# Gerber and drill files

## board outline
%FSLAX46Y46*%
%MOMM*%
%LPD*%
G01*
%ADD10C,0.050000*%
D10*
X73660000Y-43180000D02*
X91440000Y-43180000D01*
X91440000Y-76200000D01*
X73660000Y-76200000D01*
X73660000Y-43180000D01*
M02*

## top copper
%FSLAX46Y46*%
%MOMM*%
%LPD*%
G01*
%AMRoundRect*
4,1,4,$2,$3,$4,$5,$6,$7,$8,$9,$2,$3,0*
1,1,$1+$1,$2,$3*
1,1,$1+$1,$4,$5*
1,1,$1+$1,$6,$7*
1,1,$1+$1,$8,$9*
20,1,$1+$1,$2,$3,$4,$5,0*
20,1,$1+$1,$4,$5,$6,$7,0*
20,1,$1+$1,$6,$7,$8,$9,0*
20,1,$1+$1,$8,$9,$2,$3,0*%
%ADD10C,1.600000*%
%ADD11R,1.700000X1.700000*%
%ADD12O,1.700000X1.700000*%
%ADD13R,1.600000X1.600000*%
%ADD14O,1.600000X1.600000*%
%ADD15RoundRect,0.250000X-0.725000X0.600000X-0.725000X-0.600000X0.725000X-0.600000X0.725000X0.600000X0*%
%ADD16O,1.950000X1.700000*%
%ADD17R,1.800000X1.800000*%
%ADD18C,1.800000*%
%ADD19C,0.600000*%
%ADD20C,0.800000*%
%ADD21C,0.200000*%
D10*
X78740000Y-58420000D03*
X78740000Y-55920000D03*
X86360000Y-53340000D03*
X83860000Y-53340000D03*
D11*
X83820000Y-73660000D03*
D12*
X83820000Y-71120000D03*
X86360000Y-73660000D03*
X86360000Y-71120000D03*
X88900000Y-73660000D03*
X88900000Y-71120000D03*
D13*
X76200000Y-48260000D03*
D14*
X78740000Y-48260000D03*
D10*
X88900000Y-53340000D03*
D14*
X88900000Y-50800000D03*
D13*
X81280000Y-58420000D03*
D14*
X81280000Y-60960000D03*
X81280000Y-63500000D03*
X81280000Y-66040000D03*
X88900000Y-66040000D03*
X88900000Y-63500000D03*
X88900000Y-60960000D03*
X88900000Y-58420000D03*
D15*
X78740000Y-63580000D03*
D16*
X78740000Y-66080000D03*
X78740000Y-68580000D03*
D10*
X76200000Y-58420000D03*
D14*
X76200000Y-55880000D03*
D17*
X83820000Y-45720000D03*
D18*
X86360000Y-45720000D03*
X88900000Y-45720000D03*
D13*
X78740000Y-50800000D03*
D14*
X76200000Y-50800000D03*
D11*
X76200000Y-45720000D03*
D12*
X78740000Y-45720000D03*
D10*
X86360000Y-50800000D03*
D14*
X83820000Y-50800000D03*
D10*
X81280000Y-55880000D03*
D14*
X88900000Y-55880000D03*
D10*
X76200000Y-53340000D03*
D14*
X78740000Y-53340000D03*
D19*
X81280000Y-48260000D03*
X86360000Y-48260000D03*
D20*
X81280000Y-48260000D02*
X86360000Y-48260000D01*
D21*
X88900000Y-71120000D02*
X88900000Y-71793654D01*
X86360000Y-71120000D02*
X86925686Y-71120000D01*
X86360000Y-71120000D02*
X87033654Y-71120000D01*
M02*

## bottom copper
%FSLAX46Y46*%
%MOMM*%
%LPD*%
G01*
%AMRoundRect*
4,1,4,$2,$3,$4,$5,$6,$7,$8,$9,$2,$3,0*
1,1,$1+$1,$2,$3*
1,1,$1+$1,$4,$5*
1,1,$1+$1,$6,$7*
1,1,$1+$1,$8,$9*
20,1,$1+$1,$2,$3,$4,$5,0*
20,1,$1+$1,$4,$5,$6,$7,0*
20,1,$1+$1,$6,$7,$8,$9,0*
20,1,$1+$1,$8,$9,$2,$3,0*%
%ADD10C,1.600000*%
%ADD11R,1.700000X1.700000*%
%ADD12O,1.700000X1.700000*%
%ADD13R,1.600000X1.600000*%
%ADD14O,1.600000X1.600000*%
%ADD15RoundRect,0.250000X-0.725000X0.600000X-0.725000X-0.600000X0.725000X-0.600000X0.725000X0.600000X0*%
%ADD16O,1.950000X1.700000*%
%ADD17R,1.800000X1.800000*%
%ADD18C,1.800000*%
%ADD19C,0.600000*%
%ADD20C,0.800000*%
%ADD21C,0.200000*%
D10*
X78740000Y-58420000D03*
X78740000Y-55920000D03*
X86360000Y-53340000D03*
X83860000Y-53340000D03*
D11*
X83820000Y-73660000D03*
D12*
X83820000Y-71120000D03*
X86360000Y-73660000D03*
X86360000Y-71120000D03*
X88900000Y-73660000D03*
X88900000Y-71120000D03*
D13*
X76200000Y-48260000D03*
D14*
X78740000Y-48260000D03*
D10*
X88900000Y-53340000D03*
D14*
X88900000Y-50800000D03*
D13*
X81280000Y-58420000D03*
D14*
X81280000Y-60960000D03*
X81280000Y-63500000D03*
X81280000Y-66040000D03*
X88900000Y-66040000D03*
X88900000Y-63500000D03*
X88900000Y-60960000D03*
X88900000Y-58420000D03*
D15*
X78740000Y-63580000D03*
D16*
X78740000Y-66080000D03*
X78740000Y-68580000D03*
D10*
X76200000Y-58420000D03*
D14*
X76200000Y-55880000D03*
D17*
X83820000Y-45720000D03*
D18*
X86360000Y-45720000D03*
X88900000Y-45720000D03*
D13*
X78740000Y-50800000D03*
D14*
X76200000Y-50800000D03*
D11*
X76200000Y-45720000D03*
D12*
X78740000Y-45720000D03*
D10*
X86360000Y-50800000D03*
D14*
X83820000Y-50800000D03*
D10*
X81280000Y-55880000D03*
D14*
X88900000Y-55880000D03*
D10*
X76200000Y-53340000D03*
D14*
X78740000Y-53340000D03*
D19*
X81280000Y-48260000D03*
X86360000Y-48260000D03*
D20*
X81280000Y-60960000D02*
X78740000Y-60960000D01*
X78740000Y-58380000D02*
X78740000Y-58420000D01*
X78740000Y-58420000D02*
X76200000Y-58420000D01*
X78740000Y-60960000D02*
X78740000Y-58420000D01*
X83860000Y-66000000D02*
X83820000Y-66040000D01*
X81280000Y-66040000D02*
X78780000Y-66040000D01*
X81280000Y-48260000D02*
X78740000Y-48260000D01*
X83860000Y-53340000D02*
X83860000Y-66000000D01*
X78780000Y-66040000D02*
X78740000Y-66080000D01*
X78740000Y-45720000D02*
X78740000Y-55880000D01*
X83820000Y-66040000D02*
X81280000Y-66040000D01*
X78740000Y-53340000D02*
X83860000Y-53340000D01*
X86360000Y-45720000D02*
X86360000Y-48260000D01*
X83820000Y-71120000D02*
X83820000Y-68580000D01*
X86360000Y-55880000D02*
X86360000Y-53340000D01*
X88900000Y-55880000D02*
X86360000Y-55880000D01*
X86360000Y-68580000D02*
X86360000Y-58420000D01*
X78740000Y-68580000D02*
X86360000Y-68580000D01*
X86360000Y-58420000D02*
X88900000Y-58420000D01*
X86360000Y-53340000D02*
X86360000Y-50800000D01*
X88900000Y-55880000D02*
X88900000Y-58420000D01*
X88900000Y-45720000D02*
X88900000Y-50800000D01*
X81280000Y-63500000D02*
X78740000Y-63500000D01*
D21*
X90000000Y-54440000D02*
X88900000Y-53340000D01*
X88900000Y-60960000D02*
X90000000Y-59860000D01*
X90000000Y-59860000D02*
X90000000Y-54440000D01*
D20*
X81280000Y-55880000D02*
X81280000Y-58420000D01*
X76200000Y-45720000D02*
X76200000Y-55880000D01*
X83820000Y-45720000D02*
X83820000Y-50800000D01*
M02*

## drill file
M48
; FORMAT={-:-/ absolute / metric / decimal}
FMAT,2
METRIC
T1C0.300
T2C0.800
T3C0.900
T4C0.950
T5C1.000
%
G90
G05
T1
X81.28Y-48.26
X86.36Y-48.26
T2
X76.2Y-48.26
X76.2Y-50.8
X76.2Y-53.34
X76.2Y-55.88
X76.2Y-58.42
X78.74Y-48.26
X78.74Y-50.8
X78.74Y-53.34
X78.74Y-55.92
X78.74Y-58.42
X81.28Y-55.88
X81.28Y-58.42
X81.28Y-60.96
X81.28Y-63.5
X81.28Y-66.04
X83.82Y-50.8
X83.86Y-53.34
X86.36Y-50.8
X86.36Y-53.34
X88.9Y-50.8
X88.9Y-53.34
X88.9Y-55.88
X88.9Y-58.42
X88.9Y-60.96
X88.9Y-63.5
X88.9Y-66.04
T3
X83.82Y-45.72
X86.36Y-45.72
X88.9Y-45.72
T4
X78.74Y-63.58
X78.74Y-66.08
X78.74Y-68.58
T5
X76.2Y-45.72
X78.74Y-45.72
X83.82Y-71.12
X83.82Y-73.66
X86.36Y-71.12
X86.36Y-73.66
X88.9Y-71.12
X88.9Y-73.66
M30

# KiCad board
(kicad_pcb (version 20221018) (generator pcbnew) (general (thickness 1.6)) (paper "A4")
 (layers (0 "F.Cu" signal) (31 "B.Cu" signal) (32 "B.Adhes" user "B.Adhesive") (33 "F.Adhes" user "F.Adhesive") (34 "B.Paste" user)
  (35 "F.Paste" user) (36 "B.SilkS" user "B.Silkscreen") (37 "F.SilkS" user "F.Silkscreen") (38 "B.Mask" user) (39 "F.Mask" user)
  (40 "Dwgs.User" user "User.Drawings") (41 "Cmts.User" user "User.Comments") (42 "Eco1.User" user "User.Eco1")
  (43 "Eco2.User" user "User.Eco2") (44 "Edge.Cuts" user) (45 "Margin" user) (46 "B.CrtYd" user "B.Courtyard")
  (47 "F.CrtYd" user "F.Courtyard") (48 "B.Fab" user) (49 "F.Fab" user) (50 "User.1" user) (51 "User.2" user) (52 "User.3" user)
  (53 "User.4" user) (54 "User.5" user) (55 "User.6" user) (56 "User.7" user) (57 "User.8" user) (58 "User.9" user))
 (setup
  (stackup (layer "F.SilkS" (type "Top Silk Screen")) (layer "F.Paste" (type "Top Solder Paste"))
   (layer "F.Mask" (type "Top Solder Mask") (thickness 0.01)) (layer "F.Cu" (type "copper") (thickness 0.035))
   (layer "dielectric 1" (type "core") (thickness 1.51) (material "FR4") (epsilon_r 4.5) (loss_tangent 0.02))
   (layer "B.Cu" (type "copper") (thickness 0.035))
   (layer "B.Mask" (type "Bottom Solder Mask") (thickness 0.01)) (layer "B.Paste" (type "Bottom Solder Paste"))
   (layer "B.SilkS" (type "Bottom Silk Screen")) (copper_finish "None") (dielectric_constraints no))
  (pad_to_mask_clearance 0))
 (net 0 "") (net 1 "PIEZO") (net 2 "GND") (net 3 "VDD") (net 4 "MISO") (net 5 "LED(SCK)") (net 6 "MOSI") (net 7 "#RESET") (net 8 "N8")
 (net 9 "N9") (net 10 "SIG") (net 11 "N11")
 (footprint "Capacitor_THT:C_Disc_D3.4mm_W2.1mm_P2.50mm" (layer "F.Cu") (at 78.74 58.42 90)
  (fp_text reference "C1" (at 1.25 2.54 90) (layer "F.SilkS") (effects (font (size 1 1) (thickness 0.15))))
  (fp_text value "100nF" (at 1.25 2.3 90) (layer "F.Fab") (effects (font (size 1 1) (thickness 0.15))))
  (pad "1" thru_hole circle (at 0 0 90) (size 1.6 1.6) (drill 0.8) (layers "*.Cu" "*.Mask") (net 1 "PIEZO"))
  (pad "2" thru_hole circle (at 2.5 0 90) (size 1.6 1.6) (drill 0.8) (layers "*.Cu" "*.Mask") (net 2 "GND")))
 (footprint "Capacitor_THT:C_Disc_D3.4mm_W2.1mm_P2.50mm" (layer "F.Cu") (at 86.36 53.34 180)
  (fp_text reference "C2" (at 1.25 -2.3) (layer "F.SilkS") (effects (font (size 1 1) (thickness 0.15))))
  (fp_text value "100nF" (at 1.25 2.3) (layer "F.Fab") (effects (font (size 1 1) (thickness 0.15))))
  (pad "1" thru_hole circle (at 0 0 180) (size 1.6 1.6) (drill 0.8) (layers "*.Cu" "*.Mask") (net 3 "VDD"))
  (pad "2" thru_hole circle (at 2.5 0 180) (size 1.6 1.6) (drill 0.8) (layers "*.Cu" "*.Mask") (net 2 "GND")))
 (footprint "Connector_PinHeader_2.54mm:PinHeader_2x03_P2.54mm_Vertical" (layer "F.Cu") (at 83.82 73.66 90)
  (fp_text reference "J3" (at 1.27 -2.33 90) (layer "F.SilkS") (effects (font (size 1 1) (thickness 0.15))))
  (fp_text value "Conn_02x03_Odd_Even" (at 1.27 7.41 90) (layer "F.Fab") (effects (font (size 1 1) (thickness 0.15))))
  (pad "1" thru_hole rect (at 0 0 90) (size 1.7 1.7) (drill 1) (layers "*.Cu" "*.Mask") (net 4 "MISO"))
  (pad "2" thru_hole oval (at 2.54 0 90) (size 1.7 1.7) (drill 1) (layers "*.Cu" "*.Mask") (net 3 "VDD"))
  (pad "3" thru_hole oval (at 0 2.54 90) (size 1.7 1.7) (drill 1) (layers "*.Cu" "*.Mask") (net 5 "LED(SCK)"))
  (pad "4" thru_hole oval (at 2.54 2.54 90) (size 1.7 1.7) (drill 1) (layers "*.Cu" "*.Mask") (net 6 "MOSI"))
  (pad "5" thru_hole oval (at 0 5.08 90) (size 1.7 1.7) (drill 1) (layers "*.Cu" "*.Mask") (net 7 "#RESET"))
  (pad "6" thru_hole oval (at 2.54 5.08 90) (size 1.7 1.7) (drill 1) (layers "*.Cu" "*.Mask") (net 2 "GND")))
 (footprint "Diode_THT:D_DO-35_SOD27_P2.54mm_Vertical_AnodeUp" (layer "F.Cu") (at 76.2 48.26)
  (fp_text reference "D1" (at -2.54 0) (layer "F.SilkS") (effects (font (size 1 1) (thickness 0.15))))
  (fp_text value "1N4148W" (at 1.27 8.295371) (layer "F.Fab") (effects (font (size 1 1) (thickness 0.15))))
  (pad "1" thru_hole rect (at 0 0) (size 1.6 1.6) (drill 0.8) (layers "*.Cu" "*.Mask") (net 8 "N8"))
  (pad "2" thru_hole oval (at 2.54 0) (size 1.6 1.6) (drill 0.8) (layers "*.Cu" "*.Mask") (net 2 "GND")))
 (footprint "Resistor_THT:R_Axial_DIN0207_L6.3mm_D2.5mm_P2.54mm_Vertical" (layer "F.Cu") (at 88.9 53.34 90)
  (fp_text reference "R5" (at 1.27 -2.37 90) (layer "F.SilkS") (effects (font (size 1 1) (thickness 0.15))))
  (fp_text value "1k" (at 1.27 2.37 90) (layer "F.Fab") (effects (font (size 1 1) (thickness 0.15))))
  (pad "1" thru_hole circle (at 0 0 90) (size 1.6 1.6) (drill 0.8) (layers "*.Cu" "*.Mask") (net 5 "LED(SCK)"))
  (pad "2" thru_hole oval (at 2.54 0 90) (size 1.6 1.6) (drill 0.8) (layers "*.Cu" "*.Mask") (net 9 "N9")))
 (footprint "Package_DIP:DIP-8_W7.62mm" (layer "F.Cu") (at 81.28 58.42)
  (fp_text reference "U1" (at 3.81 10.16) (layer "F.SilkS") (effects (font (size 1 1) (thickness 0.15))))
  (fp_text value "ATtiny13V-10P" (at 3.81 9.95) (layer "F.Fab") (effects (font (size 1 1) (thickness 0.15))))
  (pad "1" thru_hole rect (at 0 0) (size 1.6 1.6) (drill 0.8) (layers "*.Cu" "*.Mask") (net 7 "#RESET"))
  (pad "2" thru_hole oval (at 0 2.54) (size 1.6 1.6) (drill 0.8) (layers "*.Cu" "*.Mask") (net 1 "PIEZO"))
  (pad "3" thru_hole oval (at 0 5.08) (size 1.6 1.6) (drill 0.8) (layers "*.Cu" "*.Mask") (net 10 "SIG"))
  (pad "4" thru_hole oval (at 0 7.62) (size 1.6 1.6) (drill 0.8) (layers "*.Cu" "*.Mask") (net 2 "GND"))
  (pad "5" thru_hole oval (at 7.62 7.62) (size 1.6 1.6) (drill 0.8) (layers "*.Cu" "*.Mask") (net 6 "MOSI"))
  (pad "6" thru_hole oval (at 7.62 5.08) (size 1.6 1.6) (drill 0.8) (layers "*.Cu" "*.Mask") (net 4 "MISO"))
  (pad "7" thru_hole oval (at 7.62 2.54) (size 1.6 1.6) (drill 0.8) (layers "*.Cu" "*.Mask") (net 5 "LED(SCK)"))
  (pad "8" thru_hole oval (at 7.62 0) (size 1.6 1.6) (drill 0.8) (layers "*.Cu" "*.Mask") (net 3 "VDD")))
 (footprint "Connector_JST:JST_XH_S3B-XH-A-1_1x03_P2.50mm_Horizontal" (layer "F.Cu") (at 78.74 63.58 -90)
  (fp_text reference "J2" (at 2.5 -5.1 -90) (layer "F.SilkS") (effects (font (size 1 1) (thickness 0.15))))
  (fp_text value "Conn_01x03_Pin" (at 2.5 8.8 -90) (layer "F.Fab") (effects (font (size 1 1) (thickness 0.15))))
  (pad "1" thru_hole roundrect (at 0 0 270) (size 1.7 1.95) (drill 0.95) (layers "*.Cu" "*.Mask") (roundrect_rratio 0.147059) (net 10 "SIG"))
  (pad "2" thru_hole oval (at 2.5 0 270) (size 1.7 1.95) (drill 0.95) (layers "*.Cu" "*.Mask") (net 2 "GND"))
  (pad "3" thru_hole oval (at 5 0 270) (size 1.7 1.95) (drill 0.95) (layers "*.Cu" "*.Mask") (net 3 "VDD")))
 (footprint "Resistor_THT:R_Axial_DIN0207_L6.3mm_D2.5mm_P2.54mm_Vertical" (layer "F.Cu") (at 76.2 58.42 90)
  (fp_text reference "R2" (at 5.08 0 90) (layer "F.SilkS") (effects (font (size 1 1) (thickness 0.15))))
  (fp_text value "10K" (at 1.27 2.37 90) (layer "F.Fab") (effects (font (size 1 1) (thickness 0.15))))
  (pad "1" thru_hole circle (at 0 0 90) (size 1.6 1.6) (drill 0.8) (layers "*.Cu" "*.Mask") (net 1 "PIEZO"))
  (pad "2" thru_hole oval (at 2.54 0 90) (size 1.6 1.6) (drill 0.8) (layers "*.Cu" "*.Mask") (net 8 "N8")))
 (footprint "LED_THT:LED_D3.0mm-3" (layer "F.Cu") (at 83.82 45.72)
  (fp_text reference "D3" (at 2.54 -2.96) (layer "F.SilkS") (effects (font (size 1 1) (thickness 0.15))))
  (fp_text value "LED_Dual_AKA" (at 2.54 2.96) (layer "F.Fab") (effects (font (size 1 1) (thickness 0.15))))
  (pad "1" thru_hole rect (at 0 0) (size 1.8 1.8) (drill 0.9) (layers "*.Cu" "*.Mask") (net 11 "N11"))
  (pad "2" thru_hole circle (at 2.54 0) (size 1.8 1.8) (drill 0.9) (layers "*.Cu" "*.Mask") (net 2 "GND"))
  (pad "3" thru_hole circle (at 5.08 0) (size 1.8 1.8) (drill 0.9) (layers "*.Cu" "*.Mask") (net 9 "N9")))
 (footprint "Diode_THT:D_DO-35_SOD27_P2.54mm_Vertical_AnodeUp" (layer "F.Cu") (at 78.74 50.8 180)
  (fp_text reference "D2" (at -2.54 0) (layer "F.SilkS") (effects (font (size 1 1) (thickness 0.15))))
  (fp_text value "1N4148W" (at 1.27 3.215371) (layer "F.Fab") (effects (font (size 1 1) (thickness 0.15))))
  (pad "1" thru_hole rect (at 0 0 180) (size 1.6 1.6) (drill 0.8) (layers "*.Cu" "*.Mask") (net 2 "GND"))
  (pad "2" thru_hole oval (at 2.54 0 180) (size 1.6 1.6) (drill 0.8) (layers "*.Cu" "*.Mask") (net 8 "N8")))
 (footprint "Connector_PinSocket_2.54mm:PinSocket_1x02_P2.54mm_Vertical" (layer "F.Cu") (at 76.2 45.72 90)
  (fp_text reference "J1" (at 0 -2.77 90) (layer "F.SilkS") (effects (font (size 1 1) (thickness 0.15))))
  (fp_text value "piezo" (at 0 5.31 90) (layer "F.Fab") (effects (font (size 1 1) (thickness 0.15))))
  (pad "1" thru_hole rect (at 0 0 90) (size 1.7 1.7) (drill 1) (layers "*.Cu" "*.Mask") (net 8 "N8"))
  (pad "2" thru_hole oval (at 0 2.54 90) (size 1.7 1.7) (drill 1) (layers "*.Cu" "*.Mask") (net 2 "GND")))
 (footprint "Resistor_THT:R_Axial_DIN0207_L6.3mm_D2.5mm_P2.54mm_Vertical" (layer "F.Cu") (at 86.36 50.8 180)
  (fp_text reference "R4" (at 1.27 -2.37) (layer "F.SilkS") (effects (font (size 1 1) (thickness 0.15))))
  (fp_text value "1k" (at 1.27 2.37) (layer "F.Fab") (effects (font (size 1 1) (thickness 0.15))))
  (pad "1" thru_hole circle (at 0 0 180) (size 1.6 1.6) (drill 0.8) (layers "*.Cu" "*.Mask") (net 3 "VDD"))
  (pad "2" thru_hole oval (at 2.54 0 180) (size 1.6 1.6) (drill 0.8) (layers "*.Cu" "*.Mask") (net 11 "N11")))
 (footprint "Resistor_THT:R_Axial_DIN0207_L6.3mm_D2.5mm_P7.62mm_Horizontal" (layer "F.Cu") (at 81.28 55.88)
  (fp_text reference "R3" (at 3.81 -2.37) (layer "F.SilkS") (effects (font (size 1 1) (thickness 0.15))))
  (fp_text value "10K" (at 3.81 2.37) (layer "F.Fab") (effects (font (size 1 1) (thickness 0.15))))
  (pad "1" thru_hole circle (at 0 0) (size 1.6 1.6) (drill 0.8) (layers "*.Cu" "*.Mask") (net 7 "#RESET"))
  (pad "2" thru_hole oval (at 7.62 0) (size 1.6 1.6) (drill 0.8) (layers "*.Cu" "*.Mask") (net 3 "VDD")))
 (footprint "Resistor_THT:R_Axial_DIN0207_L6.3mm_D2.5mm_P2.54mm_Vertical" (layer "F.Cu") (at 76.2 53.34)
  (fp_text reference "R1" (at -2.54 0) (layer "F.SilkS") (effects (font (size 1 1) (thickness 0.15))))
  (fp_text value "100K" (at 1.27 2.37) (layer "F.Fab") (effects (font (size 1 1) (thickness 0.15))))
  (pad "1" thru_hole circle (at 0 0) (size 1.6 1.6) (drill 0.8) (layers "*.Cu" "*.Mask") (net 8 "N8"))
  (pad "2" thru_hole oval (at 2.54 0) (size 1.6 1.6) (drill 0.8) (layers "*.Cu" "*.Mask") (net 2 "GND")))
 (gr_rect (start 73.66 43.18) (end 91.44 76.2) (stroke (width 0.05) (type default)) (fill none) (layer "Edge.Cuts"))
 (segment (start 81.28 60.96) (end 78.74 60.96) (width 0.8) (layer "B.Cu") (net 1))
 (segment (start 78.74 58.38) (end 78.74 58.42) (width 0.8) (layer "B.Cu") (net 1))
 (segment (start 78.74 58.42) (end 76.2 58.42) (width 0.8) (layer "B.Cu") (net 1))
 (segment (start 78.74 60.96) (end 78.74 58.42) (width 0.8) (layer "B.Cu") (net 1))
 (segment (start 81.28 48.26) (end 86.36 48.26) (width 0.8) (layer "F.Cu") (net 2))
 (segment (start 88.9 71.12) (end 88.9 71.793654) (width 0.2) (layer "F.Cu") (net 2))
 (via (at 81.28 48.26) (size 0.6) (drill 0.3) (layers "F.Cu" "B.Cu") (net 2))
 (via (at 86.36 48.26) (size 0.6) (drill 0.3) (layers "F.Cu" "B.Cu") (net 2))
 (segment (start 83.86 66) (end 83.82 66.04) (width 0.8) (layer "B.Cu") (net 2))
 (segment (start 81.28 66.04) (end 78.78 66.04) (width 0.8) (layer "B.Cu") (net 2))
 (segment (start 81.28 48.26) (end 78.74 48.26) (width 0.8) (layer "B.Cu") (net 2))
 (segment (start 83.86 53.34) (end 83.86 66) (width 0.8) (layer "B.Cu") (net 2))
 (segment (start 78.78 66.04) (end 78.74 66.08) (width 0.8) (layer "B.Cu") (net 2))
 (segment (start 78.74 45.72) (end 78.74 55.88) (width 0.8) (layer "B.Cu") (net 2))
 (segment (start 83.82 66.04) (end 81.28 66.04) (width 0.8) (layer "B.Cu") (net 2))
 (segment (start 78.74 53.34) (end 83.86 53.34) (width 0.8) (layer "B.Cu") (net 2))
 (segment (start 86.36 45.72) (end 86.36 48.26) (width 0.8) (layer "B.Cu") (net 2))
 (segment (start 83.82 71.12) (end 83.82 68.58) (width 0.8) (layer "B.Cu") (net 3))
 (segment (start 86.36 55.88) (end 86.36 53.34) (width 0.8) (layer "B.Cu") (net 3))
 (segment (start 88.9 55.88) (end 86.36 55.88) (width 0.8) (layer "B.Cu") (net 3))
 (segment (start 86.36 68.58) (end 86.36 58.42) (width 0.8) (layer "B.Cu") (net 3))
 (segment (start 78.74 68.58) (end 86.36 68.58) (width 0.8) (layer "B.Cu") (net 3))
 (segment (start 86.36 58.42) (end 88.9 58.42) (width 0.8) (layer "B.Cu") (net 3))
 (segment (start 86.36 53.34) (end 86.36 50.8) (width 0.8) (layer "B.Cu") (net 3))
 (segment (start 88.9 55.88) (end 88.9 58.42) (width 0.8) (layer "B.Cu") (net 3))
 (segment (start 88.9 45.72) (end 88.9 50.8) (width 0.8) (layer "B.Cu") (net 9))
 (segment (start 81.28 63.5) (end 78.74 63.5) (width 0.8) (layer "B.Cu") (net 10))
 (segment (start 90 54.44) (end 88.9 53.34) (width 0.2) (layer "B.Cu") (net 5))
 (segment (start 88.9 60.96) (end 90 59.86) (width 0.2) (layer "B.Cu") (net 5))
 (segment (start 90 59.86) (end 90 54.44) (width 0.2) (layer "B.Cu") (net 5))
 (segment (start 81.28 55.88) (end 81.28 58.42) (width 0.8) (layer "B.Cu") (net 7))
 (segment (start 86.36 71.12) (end 86.925686 71.12) (width 0.2) (layer "F.Cu") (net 6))
 (segment (start 86.36 71.12) (end 87.033654 71.12) (width 0.2) (layer "F.Cu") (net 6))
 (segment (start 76.2 45.72) (end 76.2 55.88) (width 0.8) (layer "B.Cu") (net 8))
 (segment (start 83.82 45.72) (end 83.82 50.8) (width 0.8) (layer "B.Cu") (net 11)))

